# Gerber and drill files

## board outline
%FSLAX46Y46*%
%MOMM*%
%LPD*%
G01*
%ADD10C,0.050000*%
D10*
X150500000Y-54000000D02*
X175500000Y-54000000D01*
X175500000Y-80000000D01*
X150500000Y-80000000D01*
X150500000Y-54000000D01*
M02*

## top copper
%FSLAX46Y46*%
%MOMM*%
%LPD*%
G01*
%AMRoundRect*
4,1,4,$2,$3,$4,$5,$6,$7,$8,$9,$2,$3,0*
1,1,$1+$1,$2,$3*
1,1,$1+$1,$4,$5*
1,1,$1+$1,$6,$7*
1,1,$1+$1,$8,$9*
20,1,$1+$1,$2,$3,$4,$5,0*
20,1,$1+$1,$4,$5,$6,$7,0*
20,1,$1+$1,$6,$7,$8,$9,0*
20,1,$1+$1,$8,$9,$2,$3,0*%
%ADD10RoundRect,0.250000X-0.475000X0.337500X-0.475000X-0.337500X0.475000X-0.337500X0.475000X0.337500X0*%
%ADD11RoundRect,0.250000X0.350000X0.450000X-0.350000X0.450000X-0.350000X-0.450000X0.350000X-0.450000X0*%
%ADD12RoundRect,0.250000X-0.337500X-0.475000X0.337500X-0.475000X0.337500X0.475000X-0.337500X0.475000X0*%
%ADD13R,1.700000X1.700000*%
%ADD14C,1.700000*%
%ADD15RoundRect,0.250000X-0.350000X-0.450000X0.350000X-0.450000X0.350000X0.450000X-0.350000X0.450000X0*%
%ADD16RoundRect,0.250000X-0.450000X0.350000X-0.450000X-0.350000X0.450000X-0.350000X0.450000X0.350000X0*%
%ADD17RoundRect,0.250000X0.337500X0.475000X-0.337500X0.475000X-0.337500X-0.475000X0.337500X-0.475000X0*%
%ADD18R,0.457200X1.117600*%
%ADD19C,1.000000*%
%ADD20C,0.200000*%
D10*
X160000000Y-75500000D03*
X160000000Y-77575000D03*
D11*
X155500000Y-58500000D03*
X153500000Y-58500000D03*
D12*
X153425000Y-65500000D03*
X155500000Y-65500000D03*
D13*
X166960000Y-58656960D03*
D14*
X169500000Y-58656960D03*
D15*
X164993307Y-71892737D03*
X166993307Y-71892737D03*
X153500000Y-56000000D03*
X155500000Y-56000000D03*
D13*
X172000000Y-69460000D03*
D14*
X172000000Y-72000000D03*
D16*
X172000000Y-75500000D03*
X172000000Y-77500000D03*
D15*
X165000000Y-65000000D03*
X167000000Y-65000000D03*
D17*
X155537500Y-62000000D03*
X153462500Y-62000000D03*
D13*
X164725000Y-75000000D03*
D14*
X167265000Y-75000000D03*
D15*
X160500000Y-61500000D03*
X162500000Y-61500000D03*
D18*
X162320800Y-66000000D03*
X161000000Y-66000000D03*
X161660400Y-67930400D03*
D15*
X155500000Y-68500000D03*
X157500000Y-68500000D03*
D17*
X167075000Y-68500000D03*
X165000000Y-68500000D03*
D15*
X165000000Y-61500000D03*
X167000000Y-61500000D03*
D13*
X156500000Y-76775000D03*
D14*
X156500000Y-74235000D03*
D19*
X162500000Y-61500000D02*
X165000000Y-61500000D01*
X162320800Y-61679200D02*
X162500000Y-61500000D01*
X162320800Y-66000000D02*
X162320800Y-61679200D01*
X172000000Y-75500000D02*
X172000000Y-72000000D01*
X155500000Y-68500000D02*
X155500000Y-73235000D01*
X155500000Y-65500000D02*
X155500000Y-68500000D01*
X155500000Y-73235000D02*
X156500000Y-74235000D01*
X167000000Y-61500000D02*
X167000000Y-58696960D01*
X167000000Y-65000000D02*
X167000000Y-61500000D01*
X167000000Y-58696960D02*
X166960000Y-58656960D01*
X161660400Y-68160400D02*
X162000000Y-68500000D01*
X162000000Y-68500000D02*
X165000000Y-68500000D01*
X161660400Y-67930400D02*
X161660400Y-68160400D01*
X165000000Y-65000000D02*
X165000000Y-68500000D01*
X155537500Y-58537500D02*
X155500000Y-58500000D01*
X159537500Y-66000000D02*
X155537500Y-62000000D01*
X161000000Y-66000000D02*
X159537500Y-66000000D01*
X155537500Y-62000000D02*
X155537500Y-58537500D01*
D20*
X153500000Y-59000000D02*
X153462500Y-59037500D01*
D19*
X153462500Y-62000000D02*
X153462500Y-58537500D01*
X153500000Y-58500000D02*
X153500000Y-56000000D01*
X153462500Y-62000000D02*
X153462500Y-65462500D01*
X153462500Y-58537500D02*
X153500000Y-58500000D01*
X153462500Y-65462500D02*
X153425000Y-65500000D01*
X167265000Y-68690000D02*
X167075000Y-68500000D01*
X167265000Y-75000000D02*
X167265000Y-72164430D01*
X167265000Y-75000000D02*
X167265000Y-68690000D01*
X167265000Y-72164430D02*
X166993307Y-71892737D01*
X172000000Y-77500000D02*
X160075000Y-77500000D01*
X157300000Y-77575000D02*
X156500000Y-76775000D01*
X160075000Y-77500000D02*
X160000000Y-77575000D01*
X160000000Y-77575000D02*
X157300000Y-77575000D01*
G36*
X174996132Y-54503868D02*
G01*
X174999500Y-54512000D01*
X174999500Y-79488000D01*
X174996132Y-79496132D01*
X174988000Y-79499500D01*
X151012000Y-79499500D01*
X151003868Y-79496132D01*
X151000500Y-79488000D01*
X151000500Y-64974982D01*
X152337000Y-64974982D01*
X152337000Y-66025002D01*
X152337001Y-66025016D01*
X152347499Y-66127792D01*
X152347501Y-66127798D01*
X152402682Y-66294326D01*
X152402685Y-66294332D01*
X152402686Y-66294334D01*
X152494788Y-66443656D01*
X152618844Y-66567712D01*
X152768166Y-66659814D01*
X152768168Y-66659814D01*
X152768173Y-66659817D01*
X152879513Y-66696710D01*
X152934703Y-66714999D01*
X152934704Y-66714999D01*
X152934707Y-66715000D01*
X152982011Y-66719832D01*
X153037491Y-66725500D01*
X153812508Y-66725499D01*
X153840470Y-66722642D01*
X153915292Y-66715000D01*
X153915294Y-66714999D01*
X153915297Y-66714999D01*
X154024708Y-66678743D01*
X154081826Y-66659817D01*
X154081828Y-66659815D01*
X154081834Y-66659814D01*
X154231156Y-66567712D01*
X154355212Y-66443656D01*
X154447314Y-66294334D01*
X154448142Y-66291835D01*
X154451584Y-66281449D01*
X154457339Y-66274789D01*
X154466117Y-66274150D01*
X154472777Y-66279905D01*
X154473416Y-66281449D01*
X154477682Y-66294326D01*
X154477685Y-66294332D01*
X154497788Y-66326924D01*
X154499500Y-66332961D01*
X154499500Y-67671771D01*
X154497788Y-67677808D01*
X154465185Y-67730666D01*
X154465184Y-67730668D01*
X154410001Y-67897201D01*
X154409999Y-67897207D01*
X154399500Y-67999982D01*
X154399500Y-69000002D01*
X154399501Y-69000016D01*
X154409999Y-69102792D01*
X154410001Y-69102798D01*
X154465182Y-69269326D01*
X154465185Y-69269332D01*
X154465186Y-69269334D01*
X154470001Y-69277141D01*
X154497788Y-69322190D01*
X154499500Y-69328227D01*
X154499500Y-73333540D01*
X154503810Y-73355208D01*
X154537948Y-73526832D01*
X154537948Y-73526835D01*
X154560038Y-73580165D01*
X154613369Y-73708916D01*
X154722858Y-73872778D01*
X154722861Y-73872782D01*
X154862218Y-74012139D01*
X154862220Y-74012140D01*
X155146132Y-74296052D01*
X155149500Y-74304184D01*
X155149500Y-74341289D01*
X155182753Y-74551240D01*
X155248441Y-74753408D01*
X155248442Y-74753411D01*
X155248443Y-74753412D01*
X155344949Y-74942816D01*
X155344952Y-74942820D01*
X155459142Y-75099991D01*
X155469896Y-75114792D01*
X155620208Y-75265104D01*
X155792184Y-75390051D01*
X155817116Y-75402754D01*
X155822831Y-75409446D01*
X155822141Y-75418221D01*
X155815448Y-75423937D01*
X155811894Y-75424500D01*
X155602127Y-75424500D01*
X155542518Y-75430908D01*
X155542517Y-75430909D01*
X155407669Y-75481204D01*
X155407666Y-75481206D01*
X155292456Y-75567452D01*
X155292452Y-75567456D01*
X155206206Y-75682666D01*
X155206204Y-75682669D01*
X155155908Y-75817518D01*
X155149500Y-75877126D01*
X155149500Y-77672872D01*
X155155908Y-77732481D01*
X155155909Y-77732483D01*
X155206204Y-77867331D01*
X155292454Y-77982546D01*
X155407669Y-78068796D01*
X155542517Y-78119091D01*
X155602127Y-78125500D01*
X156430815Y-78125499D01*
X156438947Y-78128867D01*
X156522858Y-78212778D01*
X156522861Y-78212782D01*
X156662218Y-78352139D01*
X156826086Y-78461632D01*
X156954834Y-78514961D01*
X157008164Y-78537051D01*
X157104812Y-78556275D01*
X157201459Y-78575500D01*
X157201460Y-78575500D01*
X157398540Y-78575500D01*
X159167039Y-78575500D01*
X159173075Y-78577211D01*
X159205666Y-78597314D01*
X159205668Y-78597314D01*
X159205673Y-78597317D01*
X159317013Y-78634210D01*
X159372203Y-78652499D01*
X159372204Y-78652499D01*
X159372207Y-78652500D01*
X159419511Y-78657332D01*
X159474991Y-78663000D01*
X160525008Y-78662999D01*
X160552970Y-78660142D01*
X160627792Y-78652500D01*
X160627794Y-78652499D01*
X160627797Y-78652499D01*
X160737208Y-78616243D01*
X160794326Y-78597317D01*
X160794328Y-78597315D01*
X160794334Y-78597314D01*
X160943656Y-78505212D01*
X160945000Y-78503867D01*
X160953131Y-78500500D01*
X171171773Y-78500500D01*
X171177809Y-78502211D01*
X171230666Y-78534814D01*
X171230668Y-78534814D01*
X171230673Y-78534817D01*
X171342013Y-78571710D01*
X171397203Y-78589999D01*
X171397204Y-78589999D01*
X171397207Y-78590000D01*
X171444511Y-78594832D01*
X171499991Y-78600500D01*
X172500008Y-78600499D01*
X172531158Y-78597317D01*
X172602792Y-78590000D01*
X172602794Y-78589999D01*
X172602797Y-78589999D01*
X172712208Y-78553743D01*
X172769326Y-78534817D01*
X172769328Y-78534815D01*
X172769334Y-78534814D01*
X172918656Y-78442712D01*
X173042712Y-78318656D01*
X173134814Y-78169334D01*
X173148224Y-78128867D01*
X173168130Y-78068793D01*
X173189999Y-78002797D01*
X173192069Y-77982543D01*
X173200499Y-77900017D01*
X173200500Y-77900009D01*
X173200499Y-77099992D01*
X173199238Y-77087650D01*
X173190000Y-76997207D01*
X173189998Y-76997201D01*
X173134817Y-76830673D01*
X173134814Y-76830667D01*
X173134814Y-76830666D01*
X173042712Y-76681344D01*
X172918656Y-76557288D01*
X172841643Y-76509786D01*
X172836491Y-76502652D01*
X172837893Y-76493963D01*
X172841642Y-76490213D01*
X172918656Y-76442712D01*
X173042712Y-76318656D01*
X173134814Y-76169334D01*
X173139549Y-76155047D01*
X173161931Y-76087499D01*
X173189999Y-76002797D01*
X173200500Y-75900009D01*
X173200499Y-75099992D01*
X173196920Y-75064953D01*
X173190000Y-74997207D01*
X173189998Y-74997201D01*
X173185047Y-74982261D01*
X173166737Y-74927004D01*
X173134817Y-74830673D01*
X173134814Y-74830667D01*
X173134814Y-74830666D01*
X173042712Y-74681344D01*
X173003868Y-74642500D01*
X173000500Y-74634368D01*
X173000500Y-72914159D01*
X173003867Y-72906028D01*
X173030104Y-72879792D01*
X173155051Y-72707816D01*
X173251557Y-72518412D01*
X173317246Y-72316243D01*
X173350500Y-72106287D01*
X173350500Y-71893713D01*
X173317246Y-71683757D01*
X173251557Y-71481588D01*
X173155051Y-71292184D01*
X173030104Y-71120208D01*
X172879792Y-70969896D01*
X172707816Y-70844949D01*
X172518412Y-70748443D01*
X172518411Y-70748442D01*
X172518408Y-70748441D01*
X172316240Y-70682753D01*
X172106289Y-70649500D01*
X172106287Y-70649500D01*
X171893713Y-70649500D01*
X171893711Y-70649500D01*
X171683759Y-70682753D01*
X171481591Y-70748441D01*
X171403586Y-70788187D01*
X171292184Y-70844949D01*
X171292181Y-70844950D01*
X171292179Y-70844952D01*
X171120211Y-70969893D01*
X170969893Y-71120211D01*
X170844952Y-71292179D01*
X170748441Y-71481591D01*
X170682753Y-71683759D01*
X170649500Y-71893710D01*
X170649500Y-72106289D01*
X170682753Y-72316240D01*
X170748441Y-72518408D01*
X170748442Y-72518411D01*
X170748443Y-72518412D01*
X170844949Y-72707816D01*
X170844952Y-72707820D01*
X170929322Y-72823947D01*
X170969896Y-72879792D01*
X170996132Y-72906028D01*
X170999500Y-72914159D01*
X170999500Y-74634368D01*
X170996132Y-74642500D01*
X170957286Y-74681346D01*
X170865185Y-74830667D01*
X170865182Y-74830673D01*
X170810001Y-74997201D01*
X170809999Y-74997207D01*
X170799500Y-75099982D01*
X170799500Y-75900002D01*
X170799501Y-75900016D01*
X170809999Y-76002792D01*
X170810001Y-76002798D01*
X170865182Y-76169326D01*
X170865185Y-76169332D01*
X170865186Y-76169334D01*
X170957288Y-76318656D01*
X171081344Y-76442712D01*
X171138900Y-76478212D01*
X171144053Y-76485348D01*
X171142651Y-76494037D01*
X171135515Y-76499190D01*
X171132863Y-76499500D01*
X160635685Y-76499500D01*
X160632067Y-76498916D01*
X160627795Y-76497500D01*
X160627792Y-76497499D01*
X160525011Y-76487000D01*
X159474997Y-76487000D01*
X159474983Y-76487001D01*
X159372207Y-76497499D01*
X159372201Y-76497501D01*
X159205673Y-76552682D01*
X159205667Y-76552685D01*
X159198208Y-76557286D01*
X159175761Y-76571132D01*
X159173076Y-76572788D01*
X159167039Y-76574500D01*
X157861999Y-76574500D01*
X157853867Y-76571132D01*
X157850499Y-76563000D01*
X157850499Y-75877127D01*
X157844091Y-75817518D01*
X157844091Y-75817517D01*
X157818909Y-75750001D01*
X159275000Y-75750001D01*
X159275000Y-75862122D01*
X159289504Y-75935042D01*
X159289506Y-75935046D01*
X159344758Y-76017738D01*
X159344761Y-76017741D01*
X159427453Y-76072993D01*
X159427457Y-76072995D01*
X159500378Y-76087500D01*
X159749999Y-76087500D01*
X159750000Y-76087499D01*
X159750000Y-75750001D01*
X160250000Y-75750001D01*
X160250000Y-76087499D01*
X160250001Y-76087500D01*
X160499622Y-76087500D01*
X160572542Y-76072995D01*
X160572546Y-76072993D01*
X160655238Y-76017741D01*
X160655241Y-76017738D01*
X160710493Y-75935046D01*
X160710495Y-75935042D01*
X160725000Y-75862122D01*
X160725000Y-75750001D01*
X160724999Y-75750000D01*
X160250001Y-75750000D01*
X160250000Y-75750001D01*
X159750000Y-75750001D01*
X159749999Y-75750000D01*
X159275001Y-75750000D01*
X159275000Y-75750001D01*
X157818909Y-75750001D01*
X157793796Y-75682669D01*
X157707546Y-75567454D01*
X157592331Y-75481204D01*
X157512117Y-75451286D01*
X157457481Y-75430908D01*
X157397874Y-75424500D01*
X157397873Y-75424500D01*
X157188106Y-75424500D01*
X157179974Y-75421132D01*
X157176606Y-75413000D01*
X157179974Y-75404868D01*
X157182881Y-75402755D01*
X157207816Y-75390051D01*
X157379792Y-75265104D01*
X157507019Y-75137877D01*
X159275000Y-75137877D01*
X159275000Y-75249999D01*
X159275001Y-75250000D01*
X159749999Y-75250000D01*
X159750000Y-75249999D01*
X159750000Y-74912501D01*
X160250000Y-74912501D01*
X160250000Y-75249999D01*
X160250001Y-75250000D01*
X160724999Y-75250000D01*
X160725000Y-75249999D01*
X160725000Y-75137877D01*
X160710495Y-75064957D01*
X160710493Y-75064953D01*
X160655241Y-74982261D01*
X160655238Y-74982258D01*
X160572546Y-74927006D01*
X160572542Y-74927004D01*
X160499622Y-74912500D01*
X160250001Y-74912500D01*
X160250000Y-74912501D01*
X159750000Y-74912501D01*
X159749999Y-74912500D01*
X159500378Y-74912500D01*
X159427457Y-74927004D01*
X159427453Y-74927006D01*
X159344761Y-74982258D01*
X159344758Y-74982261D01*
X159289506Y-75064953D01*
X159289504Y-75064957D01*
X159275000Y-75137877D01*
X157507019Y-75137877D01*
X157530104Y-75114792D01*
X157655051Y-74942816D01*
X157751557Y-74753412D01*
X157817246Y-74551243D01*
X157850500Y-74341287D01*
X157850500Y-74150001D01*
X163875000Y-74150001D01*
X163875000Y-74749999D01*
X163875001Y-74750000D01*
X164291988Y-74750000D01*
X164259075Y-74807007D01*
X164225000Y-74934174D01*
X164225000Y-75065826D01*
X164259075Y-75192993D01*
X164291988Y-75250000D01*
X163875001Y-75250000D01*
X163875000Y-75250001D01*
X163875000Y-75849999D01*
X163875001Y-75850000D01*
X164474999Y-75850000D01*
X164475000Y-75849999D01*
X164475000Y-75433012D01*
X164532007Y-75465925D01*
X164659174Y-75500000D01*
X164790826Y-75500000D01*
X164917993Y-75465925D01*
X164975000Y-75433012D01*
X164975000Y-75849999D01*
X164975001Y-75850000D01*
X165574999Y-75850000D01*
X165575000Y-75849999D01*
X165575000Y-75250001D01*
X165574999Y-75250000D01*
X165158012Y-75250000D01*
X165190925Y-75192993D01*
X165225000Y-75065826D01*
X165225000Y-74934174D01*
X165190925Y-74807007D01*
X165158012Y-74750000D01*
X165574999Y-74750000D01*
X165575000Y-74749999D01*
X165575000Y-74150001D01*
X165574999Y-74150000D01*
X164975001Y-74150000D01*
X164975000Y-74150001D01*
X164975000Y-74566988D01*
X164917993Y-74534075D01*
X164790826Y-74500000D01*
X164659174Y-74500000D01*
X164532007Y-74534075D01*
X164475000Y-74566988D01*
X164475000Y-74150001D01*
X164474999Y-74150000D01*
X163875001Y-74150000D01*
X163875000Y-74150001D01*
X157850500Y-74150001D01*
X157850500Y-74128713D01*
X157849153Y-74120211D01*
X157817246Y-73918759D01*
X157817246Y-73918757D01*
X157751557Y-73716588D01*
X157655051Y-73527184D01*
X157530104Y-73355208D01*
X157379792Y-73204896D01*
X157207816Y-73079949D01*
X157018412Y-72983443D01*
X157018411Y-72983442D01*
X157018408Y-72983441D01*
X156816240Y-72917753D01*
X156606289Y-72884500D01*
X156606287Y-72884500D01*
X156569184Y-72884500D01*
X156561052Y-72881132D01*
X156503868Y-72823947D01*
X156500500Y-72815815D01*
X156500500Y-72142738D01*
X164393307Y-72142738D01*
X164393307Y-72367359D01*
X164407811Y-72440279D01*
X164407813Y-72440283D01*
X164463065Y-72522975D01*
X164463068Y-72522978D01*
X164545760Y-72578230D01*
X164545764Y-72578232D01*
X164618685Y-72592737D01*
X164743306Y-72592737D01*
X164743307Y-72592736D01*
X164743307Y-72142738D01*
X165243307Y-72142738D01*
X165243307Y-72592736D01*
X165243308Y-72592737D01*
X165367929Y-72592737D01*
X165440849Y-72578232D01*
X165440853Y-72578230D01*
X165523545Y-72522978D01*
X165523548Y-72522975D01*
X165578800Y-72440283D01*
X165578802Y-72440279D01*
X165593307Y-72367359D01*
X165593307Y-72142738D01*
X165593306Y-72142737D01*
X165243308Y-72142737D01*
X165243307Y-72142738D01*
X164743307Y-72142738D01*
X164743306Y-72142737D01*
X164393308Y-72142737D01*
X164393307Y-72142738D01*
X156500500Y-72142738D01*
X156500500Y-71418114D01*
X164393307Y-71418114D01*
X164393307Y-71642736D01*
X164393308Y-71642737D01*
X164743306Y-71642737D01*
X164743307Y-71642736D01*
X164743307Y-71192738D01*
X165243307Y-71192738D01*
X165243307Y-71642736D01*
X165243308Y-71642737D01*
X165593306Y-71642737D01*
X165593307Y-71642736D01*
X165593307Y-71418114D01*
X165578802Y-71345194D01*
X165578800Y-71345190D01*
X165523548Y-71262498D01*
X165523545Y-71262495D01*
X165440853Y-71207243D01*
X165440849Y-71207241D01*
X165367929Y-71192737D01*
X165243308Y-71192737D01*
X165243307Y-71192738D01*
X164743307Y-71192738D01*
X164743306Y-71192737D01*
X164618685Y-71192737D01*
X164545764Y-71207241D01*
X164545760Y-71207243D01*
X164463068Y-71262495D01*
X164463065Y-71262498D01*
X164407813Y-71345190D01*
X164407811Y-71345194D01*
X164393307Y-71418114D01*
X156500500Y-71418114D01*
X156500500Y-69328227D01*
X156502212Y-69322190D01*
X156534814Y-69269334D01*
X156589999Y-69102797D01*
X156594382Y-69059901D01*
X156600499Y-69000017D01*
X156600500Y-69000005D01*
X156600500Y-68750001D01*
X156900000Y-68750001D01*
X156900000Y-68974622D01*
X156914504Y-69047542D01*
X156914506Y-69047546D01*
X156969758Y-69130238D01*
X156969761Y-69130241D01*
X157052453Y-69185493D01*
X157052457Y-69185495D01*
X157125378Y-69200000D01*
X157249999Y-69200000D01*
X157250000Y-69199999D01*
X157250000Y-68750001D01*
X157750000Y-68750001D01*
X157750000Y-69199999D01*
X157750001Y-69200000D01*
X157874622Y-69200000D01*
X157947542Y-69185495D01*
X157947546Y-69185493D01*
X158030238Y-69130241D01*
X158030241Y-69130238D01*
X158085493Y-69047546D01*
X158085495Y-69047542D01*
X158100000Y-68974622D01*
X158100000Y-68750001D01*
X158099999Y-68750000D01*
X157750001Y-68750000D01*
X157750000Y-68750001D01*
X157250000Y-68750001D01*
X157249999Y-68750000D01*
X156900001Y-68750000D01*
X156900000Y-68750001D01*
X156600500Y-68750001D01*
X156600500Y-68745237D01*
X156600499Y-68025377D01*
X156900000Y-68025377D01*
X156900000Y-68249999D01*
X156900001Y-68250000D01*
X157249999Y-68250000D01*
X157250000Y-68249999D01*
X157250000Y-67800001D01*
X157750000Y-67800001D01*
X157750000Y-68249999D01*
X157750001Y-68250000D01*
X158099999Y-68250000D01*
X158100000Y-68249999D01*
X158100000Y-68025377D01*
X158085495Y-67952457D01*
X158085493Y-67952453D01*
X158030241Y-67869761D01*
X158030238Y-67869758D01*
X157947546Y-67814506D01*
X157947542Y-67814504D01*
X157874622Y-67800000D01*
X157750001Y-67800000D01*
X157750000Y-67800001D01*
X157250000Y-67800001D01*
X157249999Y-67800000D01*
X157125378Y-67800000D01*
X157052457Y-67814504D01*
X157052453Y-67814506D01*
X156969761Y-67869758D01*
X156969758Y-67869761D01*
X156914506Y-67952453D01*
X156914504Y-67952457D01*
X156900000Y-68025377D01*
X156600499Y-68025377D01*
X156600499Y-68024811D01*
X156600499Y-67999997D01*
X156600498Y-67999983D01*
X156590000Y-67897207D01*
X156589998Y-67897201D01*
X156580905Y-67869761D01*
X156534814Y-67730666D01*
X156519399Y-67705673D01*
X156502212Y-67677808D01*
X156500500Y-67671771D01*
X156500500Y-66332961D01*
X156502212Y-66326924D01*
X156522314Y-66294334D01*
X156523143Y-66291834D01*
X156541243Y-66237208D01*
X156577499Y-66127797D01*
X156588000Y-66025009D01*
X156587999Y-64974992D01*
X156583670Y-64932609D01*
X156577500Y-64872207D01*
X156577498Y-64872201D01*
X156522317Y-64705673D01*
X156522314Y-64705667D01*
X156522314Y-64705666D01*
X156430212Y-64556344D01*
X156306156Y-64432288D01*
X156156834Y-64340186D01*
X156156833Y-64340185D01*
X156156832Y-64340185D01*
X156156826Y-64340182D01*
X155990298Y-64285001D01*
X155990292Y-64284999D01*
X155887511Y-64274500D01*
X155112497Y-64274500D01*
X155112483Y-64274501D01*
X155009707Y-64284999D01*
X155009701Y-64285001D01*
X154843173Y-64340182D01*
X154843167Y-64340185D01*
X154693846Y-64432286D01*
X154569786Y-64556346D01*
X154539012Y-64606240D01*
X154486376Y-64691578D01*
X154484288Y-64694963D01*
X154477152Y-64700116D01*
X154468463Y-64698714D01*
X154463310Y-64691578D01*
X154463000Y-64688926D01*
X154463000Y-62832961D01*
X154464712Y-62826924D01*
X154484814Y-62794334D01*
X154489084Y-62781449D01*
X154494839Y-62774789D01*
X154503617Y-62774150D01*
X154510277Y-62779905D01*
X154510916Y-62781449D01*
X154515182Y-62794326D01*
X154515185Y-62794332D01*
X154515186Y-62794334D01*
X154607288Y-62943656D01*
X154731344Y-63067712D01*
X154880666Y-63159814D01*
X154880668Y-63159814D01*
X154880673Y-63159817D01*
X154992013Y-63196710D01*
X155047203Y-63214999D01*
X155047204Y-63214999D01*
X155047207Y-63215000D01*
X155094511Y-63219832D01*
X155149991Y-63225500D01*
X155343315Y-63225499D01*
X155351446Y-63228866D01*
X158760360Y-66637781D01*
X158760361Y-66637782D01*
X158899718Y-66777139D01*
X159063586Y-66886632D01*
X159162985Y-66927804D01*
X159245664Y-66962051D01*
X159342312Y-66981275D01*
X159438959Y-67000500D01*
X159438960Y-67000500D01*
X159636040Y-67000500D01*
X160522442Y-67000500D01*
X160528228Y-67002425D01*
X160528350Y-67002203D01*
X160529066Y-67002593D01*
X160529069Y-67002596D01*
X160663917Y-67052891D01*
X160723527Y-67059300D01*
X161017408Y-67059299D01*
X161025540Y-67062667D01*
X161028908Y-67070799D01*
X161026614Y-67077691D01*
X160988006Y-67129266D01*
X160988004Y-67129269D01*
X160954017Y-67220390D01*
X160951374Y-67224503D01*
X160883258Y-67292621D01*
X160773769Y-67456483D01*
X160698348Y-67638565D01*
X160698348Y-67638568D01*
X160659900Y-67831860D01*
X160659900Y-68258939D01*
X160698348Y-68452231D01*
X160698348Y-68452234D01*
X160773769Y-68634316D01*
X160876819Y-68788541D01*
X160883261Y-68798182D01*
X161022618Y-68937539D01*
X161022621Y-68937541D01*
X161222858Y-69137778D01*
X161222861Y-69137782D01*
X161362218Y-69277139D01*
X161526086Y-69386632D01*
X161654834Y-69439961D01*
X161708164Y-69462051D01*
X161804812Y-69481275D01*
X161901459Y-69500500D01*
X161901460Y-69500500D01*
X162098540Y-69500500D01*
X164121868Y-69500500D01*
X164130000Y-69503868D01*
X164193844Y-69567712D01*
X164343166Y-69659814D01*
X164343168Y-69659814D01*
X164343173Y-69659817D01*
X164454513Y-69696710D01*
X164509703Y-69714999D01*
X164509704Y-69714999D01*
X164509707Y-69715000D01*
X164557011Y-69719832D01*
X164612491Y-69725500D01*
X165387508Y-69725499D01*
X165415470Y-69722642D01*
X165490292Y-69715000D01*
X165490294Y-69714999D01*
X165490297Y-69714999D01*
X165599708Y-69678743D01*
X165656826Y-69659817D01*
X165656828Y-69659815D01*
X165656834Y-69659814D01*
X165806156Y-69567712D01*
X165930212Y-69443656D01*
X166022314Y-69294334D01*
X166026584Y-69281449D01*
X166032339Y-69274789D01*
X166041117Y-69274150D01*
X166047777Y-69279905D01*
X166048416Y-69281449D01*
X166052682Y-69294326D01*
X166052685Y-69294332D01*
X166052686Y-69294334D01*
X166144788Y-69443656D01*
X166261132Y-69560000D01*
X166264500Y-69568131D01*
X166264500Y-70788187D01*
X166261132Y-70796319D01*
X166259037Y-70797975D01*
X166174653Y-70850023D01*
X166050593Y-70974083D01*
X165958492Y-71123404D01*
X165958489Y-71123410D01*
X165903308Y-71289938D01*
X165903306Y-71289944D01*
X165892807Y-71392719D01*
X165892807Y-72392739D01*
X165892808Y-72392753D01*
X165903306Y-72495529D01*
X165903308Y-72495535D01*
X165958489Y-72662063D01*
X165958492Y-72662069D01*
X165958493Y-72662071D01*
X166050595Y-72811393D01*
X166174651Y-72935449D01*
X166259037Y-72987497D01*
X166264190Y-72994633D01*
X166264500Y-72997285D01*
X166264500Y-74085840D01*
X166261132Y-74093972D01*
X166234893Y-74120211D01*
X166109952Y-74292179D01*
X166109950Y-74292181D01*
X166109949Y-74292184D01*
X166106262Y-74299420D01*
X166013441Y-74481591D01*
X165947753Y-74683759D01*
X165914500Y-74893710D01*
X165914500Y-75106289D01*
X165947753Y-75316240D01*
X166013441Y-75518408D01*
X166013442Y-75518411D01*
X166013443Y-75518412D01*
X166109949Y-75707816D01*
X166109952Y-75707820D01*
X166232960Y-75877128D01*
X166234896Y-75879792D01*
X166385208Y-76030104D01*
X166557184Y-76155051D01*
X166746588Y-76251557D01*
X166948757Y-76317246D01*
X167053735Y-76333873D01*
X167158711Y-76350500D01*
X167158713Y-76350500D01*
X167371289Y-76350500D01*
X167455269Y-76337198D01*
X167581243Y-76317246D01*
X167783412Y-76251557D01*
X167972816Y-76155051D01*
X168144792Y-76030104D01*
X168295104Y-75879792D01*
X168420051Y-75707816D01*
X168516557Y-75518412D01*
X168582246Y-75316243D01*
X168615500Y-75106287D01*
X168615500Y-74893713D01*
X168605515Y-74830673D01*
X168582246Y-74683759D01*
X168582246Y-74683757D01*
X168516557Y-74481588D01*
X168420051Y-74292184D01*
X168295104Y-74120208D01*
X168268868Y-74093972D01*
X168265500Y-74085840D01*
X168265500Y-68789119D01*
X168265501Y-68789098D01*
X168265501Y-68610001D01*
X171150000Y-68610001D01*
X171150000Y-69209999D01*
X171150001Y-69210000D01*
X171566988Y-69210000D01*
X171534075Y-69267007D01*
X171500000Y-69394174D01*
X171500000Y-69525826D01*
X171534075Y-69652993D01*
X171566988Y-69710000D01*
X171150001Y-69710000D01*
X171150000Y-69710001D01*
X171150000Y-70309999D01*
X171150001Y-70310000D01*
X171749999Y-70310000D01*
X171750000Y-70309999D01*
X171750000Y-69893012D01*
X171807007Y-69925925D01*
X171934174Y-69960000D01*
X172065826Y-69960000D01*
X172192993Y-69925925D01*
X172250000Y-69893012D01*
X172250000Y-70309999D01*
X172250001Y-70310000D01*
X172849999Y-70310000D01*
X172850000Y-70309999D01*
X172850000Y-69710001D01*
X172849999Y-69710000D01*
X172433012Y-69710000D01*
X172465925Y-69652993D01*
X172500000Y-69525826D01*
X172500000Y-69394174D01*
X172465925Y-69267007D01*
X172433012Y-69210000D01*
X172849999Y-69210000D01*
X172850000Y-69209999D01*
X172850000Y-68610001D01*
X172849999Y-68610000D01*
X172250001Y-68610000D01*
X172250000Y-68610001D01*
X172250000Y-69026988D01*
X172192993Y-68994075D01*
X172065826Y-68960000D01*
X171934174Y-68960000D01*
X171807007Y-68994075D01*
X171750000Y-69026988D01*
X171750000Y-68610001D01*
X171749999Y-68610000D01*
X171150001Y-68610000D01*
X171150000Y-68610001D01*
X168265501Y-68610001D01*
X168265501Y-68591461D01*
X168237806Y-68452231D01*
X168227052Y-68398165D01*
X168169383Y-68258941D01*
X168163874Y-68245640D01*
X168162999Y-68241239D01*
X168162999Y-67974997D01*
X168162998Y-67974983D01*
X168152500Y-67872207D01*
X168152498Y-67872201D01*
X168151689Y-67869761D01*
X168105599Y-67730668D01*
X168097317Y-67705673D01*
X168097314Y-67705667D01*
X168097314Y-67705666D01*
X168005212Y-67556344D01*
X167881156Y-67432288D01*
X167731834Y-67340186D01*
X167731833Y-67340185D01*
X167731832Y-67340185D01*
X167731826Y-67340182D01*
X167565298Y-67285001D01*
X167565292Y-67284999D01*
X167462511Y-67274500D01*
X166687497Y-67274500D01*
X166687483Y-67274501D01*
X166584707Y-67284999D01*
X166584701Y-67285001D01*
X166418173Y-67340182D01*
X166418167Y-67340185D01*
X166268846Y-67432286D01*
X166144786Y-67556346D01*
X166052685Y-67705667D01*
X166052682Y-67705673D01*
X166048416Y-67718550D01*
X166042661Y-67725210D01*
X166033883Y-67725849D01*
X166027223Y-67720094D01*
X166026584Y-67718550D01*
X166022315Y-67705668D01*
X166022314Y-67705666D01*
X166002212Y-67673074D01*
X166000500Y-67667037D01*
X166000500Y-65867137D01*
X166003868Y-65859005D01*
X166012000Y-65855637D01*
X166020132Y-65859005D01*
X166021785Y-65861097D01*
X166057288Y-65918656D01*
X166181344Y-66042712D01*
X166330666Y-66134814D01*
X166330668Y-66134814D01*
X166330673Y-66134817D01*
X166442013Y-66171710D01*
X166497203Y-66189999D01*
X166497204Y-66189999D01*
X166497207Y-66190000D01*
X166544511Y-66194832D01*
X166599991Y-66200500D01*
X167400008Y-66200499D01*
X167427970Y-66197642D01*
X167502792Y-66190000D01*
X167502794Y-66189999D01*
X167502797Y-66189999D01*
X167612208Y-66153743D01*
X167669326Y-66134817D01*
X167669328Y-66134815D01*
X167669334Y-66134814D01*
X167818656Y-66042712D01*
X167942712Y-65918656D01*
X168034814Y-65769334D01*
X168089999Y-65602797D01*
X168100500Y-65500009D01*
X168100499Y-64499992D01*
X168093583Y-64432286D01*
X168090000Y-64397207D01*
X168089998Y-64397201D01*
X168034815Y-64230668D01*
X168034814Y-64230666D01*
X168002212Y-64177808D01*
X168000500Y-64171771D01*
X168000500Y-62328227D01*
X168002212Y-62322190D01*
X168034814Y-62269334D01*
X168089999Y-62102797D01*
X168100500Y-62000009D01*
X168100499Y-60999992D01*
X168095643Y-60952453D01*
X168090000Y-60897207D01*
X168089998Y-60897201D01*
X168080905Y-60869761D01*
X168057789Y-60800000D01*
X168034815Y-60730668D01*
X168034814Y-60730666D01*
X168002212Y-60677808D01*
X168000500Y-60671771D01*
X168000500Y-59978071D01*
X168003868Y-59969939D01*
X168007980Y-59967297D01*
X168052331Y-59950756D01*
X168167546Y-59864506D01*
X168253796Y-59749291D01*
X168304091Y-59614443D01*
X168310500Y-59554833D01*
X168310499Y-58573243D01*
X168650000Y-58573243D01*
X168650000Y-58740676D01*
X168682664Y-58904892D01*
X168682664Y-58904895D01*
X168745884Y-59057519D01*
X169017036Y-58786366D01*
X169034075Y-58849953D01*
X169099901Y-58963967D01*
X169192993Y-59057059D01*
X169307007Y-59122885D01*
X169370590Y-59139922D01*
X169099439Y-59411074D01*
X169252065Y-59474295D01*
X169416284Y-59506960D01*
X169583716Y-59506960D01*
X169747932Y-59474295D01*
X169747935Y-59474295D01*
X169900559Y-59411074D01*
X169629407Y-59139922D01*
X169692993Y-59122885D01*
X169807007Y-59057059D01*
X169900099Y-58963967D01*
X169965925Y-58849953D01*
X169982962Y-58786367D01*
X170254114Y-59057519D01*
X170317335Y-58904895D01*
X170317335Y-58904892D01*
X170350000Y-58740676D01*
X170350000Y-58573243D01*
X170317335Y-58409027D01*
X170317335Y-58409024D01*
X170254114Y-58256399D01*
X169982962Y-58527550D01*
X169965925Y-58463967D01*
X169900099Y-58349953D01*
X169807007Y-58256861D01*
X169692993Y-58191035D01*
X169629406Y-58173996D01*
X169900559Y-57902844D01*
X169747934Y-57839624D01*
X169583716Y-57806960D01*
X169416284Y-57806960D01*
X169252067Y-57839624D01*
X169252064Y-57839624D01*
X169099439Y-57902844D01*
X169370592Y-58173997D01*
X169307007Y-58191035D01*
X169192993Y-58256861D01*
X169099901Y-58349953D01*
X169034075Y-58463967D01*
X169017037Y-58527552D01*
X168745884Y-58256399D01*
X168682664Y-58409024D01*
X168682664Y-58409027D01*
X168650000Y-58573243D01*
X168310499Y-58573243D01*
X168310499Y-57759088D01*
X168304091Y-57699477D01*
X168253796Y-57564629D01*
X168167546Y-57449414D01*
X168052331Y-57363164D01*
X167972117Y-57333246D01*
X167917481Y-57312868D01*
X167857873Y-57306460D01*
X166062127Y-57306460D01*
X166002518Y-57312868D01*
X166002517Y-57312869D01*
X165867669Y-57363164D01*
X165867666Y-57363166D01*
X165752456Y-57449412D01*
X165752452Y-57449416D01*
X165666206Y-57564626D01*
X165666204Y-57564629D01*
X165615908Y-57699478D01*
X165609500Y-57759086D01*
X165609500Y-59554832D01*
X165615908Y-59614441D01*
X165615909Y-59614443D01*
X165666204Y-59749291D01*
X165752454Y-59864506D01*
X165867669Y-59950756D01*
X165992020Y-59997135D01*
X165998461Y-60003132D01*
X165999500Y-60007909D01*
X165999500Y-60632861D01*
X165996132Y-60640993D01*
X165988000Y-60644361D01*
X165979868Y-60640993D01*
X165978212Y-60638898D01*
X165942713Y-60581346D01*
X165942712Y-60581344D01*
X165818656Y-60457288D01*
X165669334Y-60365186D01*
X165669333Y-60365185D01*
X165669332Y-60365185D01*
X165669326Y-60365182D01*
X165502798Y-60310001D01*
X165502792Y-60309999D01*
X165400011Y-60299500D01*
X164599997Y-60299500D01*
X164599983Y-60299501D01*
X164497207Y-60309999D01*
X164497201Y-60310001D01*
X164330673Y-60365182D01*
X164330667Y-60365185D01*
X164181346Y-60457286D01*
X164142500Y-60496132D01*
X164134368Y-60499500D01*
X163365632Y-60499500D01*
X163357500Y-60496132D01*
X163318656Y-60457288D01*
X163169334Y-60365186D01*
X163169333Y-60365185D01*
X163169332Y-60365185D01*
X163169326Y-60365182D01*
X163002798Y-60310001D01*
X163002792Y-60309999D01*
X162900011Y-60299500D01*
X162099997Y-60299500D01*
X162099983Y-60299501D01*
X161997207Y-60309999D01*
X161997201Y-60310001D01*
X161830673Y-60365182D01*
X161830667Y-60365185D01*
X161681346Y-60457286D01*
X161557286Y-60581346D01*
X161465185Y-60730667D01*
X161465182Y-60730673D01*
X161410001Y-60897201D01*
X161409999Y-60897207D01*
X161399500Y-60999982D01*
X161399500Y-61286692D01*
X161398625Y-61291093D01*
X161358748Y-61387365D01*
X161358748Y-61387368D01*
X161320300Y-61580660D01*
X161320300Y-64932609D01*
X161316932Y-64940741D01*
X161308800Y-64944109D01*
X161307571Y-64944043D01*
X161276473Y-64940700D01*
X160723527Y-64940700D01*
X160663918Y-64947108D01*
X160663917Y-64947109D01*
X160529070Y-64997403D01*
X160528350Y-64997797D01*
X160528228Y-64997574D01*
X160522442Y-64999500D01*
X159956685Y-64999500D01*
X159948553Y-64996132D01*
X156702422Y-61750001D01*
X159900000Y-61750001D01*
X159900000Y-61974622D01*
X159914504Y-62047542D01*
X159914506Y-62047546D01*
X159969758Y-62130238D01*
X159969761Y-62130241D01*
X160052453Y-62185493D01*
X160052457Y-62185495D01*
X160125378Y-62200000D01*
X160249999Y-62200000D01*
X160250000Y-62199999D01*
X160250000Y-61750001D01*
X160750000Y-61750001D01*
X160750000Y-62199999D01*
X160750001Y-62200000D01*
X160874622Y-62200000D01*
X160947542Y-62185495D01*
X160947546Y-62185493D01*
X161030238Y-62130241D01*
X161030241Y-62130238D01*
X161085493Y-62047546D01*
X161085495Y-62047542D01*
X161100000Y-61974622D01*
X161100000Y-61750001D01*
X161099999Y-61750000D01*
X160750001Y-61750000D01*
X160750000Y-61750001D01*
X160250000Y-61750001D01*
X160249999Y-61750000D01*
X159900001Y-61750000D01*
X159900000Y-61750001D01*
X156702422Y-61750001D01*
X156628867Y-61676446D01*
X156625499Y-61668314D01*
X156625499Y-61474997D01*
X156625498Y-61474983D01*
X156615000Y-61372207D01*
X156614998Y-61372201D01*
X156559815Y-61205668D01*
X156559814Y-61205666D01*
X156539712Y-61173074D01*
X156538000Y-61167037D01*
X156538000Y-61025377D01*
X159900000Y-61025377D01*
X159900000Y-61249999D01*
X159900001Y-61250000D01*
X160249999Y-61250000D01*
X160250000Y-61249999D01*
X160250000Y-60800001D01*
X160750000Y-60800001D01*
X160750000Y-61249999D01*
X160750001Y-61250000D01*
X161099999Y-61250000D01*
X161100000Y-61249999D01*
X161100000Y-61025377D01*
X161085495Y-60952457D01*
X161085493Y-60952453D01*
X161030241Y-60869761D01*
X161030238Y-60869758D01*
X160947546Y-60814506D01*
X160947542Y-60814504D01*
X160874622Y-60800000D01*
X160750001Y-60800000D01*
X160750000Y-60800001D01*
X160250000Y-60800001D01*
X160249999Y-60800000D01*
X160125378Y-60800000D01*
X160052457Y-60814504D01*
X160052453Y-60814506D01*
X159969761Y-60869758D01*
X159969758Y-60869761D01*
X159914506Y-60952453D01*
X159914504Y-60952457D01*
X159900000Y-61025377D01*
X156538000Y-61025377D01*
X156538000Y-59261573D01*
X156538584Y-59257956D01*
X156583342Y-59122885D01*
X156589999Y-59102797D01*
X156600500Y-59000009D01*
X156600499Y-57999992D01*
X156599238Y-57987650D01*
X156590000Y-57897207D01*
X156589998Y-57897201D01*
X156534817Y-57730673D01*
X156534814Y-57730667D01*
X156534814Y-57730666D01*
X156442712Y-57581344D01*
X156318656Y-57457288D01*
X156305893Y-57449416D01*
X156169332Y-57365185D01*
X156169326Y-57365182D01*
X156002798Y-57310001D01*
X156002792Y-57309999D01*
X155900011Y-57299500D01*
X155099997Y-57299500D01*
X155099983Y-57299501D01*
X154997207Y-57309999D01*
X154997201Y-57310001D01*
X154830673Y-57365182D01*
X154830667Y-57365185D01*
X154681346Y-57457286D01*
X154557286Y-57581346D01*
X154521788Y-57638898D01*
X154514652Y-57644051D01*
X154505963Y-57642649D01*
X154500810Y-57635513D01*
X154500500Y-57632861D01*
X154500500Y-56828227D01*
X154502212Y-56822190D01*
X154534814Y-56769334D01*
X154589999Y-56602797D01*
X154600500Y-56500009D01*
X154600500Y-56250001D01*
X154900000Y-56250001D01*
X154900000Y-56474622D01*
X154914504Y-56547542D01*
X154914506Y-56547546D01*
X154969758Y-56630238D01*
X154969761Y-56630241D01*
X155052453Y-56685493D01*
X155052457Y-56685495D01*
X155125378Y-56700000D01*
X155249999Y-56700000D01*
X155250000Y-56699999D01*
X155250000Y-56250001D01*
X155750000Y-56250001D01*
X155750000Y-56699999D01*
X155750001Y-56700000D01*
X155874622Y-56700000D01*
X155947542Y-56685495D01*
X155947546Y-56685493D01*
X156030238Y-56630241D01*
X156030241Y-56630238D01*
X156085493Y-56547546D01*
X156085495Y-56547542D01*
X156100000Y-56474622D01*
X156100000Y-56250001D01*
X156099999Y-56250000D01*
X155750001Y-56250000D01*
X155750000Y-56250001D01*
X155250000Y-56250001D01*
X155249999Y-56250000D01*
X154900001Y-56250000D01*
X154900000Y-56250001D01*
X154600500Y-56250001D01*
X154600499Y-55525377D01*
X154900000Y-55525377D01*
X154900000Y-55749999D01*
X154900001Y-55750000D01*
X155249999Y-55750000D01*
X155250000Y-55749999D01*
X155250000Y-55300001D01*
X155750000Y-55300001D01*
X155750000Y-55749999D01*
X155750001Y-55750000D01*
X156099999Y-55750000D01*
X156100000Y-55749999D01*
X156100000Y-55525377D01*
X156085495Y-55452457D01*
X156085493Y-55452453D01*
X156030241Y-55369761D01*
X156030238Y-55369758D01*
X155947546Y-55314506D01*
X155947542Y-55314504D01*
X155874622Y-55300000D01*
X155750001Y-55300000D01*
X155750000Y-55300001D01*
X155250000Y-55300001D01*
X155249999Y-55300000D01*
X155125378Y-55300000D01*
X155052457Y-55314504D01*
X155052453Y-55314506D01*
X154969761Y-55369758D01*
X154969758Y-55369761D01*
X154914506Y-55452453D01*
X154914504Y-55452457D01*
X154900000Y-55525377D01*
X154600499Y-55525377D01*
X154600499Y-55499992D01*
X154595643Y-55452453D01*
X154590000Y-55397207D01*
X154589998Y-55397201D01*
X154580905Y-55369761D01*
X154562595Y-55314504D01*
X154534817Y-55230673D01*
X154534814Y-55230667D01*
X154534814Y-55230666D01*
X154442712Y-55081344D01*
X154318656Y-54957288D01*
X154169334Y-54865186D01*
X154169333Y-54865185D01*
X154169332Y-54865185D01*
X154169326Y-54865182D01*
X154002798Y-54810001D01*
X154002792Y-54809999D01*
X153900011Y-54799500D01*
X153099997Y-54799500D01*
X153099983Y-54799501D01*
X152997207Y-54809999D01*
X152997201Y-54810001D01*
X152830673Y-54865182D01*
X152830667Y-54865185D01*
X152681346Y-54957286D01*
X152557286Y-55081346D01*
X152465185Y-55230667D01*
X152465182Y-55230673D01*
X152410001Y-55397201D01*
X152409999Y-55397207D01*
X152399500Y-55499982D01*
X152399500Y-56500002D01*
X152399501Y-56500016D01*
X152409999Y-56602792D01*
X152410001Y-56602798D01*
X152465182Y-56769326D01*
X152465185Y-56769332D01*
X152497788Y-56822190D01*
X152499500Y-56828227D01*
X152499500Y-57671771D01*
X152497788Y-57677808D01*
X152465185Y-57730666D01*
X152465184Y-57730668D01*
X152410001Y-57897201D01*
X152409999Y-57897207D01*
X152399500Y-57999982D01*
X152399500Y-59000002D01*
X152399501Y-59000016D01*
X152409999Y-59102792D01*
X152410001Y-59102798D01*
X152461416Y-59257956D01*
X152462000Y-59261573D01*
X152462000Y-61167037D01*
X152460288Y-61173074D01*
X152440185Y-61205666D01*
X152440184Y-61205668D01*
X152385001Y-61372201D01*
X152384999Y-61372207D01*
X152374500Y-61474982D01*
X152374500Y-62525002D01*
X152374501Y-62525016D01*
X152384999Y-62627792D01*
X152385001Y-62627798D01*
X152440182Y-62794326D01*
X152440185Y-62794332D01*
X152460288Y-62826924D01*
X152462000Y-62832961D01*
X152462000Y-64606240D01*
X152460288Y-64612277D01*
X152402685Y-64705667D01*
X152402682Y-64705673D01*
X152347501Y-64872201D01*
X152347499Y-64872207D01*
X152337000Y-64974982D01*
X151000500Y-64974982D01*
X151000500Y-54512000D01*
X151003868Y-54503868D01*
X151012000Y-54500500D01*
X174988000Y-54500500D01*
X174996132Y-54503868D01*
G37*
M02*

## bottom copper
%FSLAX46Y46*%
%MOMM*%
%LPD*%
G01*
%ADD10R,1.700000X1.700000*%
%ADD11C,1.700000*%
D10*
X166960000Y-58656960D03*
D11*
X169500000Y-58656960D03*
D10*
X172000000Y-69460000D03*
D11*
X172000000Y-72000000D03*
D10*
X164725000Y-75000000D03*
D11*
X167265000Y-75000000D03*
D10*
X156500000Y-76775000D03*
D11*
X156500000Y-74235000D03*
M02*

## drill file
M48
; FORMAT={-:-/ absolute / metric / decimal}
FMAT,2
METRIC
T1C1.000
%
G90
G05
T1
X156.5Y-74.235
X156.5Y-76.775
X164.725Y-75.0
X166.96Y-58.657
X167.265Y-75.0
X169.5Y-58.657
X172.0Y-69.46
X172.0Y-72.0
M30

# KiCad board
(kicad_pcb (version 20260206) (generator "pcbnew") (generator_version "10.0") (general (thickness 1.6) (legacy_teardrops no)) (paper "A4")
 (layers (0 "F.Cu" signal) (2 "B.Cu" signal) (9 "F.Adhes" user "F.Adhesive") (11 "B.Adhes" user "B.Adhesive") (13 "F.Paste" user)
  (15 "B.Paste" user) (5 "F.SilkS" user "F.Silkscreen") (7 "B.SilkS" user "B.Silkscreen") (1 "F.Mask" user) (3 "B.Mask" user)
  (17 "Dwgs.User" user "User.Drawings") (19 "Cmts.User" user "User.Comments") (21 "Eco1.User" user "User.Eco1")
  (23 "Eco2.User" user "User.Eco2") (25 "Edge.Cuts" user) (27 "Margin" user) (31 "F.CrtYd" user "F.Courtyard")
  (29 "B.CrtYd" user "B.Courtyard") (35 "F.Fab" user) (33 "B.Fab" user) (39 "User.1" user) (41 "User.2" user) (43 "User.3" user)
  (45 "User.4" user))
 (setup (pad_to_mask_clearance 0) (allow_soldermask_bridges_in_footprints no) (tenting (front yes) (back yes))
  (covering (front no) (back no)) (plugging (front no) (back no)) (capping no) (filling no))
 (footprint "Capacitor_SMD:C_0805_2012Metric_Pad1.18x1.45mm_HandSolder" (layer "F.Cu") (at 160 76.5375 -90)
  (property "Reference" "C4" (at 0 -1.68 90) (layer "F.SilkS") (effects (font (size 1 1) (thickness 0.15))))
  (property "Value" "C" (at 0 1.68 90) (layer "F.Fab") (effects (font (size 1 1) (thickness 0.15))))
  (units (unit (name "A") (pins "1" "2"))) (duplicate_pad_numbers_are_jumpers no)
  (pad "1" smd roundrect (at -1.0375 0 270) (size 1.175 1.45) (layers "F.Cu" "F.Mask" "F.Paste") (roundrect_rratio 0.212766) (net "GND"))
  (pad "2" smd roundrect (at 1.0375 0 270) (size 1.175 1.45) (layers "F.Cu" "F.Mask" "F.Paste") (roundrect_rratio 0.212766)
   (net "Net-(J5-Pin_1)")))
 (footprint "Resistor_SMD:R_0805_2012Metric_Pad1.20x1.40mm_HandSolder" (layer "F.Cu") (at 154.5 58.5 180)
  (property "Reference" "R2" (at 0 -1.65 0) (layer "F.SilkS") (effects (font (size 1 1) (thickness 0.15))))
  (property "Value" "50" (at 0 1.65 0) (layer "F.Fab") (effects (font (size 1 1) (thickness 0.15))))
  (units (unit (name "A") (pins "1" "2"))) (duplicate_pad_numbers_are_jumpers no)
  (pad "1" smd roundrect (at -1 0 180) (size 1.2 1.4) (layers "F.Cu" "F.Mask" "F.Paste") (roundrect_rratio 0.208333) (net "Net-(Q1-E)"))
  (pad "2" smd roundrect (at 1 0 180) (size 1.2 1.4) (layers "F.Cu" "F.Mask" "F.Paste") (roundrect_rratio 0.208333) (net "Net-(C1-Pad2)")))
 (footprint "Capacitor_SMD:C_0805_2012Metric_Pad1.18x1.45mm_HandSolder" (layer "F.Cu") (at 154.4625 65.5)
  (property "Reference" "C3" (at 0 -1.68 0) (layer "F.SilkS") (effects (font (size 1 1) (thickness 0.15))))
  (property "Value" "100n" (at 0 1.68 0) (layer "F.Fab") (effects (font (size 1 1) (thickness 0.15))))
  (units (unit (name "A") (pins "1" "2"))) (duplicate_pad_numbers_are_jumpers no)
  (pad "1" smd roundrect (at -1.0375 0) (size 1.175 1.45) (layers "F.Cu" "F.Mask" "F.Paste") (roundrect_rratio 0.212766)
   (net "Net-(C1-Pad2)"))
  (pad "2" smd roundrect (at 1.0375 0) (size 1.175 1.45) (layers "F.Cu" "F.Mask" "F.Paste") (roundrect_rratio 0.212766)
   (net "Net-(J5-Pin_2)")))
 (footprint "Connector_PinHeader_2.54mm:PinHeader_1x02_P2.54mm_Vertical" (layer "F.Cu") (at 166.96 58.65696 90)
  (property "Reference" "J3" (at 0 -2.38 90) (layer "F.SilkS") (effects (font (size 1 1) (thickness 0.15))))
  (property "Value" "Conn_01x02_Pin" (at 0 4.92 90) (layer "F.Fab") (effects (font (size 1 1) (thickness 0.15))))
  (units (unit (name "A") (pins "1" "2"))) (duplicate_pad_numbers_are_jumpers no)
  (pad "1" thru_hole rect (at 0 0 90) (size 1.7 1.7) (drill 1) (layers "*.Cu" "*.Mask") (remove_unused_layers no) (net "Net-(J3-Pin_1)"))
  (pad "2" thru_hole circle (at 0 2.54 90) (size 1.7 1.7) (drill 1) (layers "*.Cu" "*.Mask") (remove_unused_layers no) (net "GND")))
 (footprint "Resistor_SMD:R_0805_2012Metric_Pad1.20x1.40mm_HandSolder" (layer "F.Cu") (at 165.993307 71.892737)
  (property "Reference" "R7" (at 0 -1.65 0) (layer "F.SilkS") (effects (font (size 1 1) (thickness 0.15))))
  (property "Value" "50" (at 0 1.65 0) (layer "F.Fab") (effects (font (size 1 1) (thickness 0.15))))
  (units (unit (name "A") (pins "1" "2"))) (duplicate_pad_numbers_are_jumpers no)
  (pad "1" smd roundrect (at -1 0) (size 1.2 1.4) (layers "F.Cu" "F.Mask" "F.Paste") (roundrect_rratio 0.208333) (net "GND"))
  (pad "2" smd roundrect (at 1 0) (size 1.2 1.4) (layers "F.Cu" "F.Mask" "F.Paste") (roundrect_rratio 0.208333) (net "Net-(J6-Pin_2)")))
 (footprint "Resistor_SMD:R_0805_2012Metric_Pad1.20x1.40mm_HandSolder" (layer "F.Cu") (at 154.5 56)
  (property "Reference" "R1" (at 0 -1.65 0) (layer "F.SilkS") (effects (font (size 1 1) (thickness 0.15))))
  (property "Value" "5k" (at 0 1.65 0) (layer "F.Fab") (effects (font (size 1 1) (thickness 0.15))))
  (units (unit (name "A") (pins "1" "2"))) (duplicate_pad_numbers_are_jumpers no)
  (pad "1" smd roundrect (at -1 0) (size 1.2 1.4) (layers "F.Cu" "F.Mask" "F.Paste") (roundrect_rratio 0.208333) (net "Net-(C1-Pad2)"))
  (pad "2" smd roundrect (at 1 0) (size 1.2 1.4) (layers "F.Cu" "F.Mask" "F.Paste") (roundrect_rratio 0.208333) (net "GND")))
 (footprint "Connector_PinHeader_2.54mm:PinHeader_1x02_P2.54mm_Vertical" (layer "F.Cu") (at 172 69.46)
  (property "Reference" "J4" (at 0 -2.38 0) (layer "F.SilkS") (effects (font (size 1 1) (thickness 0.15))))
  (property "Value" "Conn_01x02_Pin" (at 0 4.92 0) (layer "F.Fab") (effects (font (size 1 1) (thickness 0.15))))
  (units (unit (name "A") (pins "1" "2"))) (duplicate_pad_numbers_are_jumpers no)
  (pad "1" thru_hole rect (at 0 0) (size 1.7 1.7) (drill 1) (layers "*.Cu" "*.Mask") (remove_unused_layers no) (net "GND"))
  (pad "2" thru_hole circle (at 0 2.54) (size 1.7 1.7) (drill 1) (layers "*.Cu" "*.Mask") (remove_unused_layers no) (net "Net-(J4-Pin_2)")))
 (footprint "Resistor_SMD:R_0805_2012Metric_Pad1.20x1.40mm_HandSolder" (layer "F.Cu") (at 172 76.5 -90)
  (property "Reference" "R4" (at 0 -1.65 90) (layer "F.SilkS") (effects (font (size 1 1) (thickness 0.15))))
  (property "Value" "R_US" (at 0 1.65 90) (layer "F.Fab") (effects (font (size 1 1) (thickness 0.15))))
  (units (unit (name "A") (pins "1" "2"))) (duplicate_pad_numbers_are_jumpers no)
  (pad "1" smd roundrect (at -1 0 270) (size 1.2 1.4) (layers "F.Cu" "F.Mask" "F.Paste") (roundrect_rratio 0.208333) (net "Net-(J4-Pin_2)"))
  (pad "2" smd roundrect (at 1 0 270) (size 1.2 1.4) (layers "F.Cu" "F.Mask" "F.Paste") (roundrect_rratio 0.208333) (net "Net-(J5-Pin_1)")))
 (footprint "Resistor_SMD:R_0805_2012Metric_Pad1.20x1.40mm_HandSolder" (layer "F.Cu") (at 166 65)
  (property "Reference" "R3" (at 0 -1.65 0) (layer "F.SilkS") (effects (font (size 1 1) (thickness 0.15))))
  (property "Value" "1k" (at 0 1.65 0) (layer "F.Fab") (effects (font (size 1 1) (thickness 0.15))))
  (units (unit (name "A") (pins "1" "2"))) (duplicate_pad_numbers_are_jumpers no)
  (pad "1" smd roundrect (at -1 0) (size 1.2 1.4) (layers "F.Cu" "F.Mask" "F.Paste") (roundrect_rratio 0.208333) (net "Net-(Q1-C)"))
  (pad "2" smd roundrect (at 1 0) (size 1.2 1.4) (layers "F.Cu" "F.Mask" "F.Paste") (roundrect_rratio 0.208333) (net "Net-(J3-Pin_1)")))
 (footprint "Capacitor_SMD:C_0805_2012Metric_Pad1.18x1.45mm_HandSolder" (layer "F.Cu") (at 154.5 62 180)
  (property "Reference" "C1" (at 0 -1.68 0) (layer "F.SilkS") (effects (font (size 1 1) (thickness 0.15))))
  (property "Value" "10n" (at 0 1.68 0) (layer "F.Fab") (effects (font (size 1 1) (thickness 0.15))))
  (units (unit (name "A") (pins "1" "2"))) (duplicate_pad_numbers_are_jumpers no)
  (pad "1" smd roundrect (at -1.0375 0 180) (size 1.175 1.45) (layers "F.Cu" "F.Mask" "F.Paste") (roundrect_rratio 0.212766)
   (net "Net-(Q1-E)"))
  (pad "2" smd roundrect (at 1.0375 0 180) (size 1.175 1.45) (layers "F.Cu" "F.Mask" "F.Paste") (roundrect_rratio 0.212766)
   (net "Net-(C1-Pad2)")))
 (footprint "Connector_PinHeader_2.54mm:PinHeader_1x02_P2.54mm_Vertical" (layer "F.Cu") (at 164.725 75 90)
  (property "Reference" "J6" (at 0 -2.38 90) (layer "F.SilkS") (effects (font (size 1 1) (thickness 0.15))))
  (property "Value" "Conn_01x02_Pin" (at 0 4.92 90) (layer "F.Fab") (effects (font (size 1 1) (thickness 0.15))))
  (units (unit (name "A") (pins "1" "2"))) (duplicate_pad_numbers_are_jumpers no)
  (pad "1" thru_hole rect (at 0 0 90) (size 1.7 1.7) (drill 1) (layers "*.Cu" "*.Mask") (remove_unused_layers no) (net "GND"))
  (pad "2" thru_hole circle (at 0 2.54 90) (size 1.7 1.7) (drill 1) (layers "*.Cu" "*.Mask") (remove_unused_layers no)
   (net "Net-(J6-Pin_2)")))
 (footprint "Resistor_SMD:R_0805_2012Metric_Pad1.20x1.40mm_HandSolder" (layer "F.Cu") (at 161.5 61.5)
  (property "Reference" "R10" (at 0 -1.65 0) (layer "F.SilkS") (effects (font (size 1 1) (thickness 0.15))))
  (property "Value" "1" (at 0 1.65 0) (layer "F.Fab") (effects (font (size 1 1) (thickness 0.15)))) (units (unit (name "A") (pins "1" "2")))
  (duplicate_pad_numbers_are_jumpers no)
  (pad "1" smd roundrect (at -1 0) (size 1.2 1.4) (layers "F.Cu" "F.Mask" "F.Paste") (roundrect_rratio 0.208333) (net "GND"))
  (pad "2" smd roundrect (at 1 0) (size 1.2 1.4) (layers "F.Cu" "F.Mask" "F.Paste") (roundrect_rratio 0.208333) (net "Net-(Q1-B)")))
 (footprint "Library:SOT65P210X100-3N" (layer "F.Cu") (at 161.6604 66.9652 -90)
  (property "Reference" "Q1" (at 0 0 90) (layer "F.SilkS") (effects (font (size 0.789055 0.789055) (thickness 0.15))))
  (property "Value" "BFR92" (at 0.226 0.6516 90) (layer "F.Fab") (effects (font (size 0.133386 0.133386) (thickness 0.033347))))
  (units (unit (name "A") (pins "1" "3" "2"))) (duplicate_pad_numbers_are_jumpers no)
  (pad "1" smd rect (at -0.9652 -0.6604 270) (size 1.1176 0.4572) (layers "F.Cu" "F.Mask" "F.Paste") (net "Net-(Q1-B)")
   (solder_mask_margin 0.102))
  (pad "2" smd rect (at -0.9652 0.6604 270) (size 1.1176 0.4572) (layers "F.Cu" "F.Mask" "F.Paste") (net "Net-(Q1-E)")
   (solder_mask_margin 0.102))
  (pad "3" smd rect (at 0.9652 0 270) (size 1.1176 0.4572) (layers "F.Cu" "F.Mask" "F.Paste") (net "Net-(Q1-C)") (solder_mask_margin 0.102)))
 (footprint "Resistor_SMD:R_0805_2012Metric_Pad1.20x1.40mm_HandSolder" (layer "F.Cu") (at 156.5 68.5)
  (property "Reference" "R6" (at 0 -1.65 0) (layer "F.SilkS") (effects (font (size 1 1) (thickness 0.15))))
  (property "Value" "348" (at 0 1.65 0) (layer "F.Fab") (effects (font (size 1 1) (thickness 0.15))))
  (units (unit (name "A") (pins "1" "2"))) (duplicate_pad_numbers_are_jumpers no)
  (pad "1" smd roundrect (at -1 0) (size 1.2 1.4) (layers "F.Cu" "F.Mask" "F.Paste") (roundrect_rratio 0.208333) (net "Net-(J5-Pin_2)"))
  (pad "2" smd roundrect (at 1 0) (size 1.2 1.4) (layers "F.Cu" "F.Mask" "F.Paste") (roundrect_rratio 0.208333) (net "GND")))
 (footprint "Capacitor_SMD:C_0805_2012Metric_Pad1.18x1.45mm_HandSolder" (layer "F.Cu") (at 166.0375 68.5 180)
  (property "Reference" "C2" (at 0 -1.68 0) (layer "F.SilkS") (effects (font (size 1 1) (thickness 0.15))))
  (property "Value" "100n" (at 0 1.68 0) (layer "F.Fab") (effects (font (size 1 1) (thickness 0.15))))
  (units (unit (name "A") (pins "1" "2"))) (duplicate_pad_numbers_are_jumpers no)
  (pad "1" smd roundrect (at -1.0375 0 180) (size 1.175 1.45) (layers "F.Cu" "F.Mask" "F.Paste") (roundrect_rratio 0.212766)
   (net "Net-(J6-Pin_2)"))
  (pad "2" smd roundrect (at 1.0375 0 180) (size 1.175 1.45) (layers "F.Cu" "F.Mask" "F.Paste") (roundrect_rratio 0.212766)
   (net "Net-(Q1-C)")))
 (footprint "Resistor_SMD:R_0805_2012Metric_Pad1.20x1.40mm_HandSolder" (layer "F.Cu") (at 166 61.5)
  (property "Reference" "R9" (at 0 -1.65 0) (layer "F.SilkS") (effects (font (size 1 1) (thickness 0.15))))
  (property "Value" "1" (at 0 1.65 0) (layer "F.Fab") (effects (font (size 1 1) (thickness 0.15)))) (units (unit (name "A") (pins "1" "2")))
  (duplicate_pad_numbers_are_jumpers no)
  (pad "1" smd roundrect (at -1 0) (size 1.2 1.4) (layers "F.Cu" "F.Mask" "F.Paste") (roundrect_rratio 0.208333) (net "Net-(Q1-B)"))
  (pad "2" smd roundrect (at 1 0) (size 1.2 1.4) (layers "F.Cu" "F.Mask" "F.Paste") (roundrect_rratio 0.208333) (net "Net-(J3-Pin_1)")))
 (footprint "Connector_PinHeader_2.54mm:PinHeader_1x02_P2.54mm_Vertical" (layer "F.Cu") (at 156.5 76.775 180)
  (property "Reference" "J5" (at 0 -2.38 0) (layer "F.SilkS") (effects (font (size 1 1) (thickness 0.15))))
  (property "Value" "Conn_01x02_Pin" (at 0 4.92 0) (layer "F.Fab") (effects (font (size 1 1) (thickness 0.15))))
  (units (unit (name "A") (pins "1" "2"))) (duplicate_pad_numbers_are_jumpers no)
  (pad "1" thru_hole rect (at 0 0 180) (size 1.7 1.7) (drill 1) (layers "*.Cu" "*.Mask") (remove_unused_layers no) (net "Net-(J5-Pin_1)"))
  (pad "2" thru_hole circle (at 0 2.54 180) (size 1.7 1.7) (drill 1) (layers "*.Cu" "*.Mask") (remove_unused_layers no)
   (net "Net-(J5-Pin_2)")))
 (gr_rect (start 150.5 54) (end 175.5 80) (stroke (width 0.05) (type default)) (fill no) (layer "Edge.Cuts"))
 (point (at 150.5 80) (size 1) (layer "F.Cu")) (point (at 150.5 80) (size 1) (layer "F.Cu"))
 (segment (start 162.5 61.5) (end 165 61.5) (width 1) (layer "F.Cu") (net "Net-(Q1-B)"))
 (segment (start 162.3208 61.6792) (end 162.5 61.5) (width 1) (layer "F.Cu") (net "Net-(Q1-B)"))
 (segment (start 162.3208 66) (end 162.3208 61.6792) (width 1) (layer "F.Cu") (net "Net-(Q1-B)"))
 (segment (start 172 75.5) (end 172 72) (width 1) (layer "F.Cu") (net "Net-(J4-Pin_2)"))
 (segment (start 155.5 68.5) (end 155.5 73.235) (width 1) (layer "F.Cu") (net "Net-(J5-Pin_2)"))
 (segment (start 155.5 65.5) (end 155.5 68.5) (width 1) (layer "F.Cu") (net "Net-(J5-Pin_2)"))
 (segment (start 155.5 73.235) (end 156.5 74.235) (width 1) (layer "F.Cu") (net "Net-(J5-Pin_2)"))
 (segment (start 167 61.5) (end 167 58.69696) (width 1) (layer "F.Cu") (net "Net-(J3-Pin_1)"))
 (segment (start 167 65) (end 167 61.5) (width 1) (layer "F.Cu") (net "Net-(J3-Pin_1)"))
 (segment (start 167 58.69696) (end 166.96 58.65696) (width 1) (layer "F.Cu") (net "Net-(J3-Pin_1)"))
 (segment (start 161.6604 68.1604) (end 162 68.5) (width 1) (layer "F.Cu") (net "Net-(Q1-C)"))
 (segment (start 162 68.5) (end 165 68.5) (width 1) (layer "F.Cu") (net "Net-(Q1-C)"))
 (segment (start 161.6604 67.9304) (end 161.6604 68.1604) (width 1) (layer "F.Cu") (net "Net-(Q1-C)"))
 (segment (start 165 65) (end 165 68.5) (width 1) (layer "F.Cu") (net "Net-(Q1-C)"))
 (segment (start 155.5375 58.5375) (end 155.5 58.5) (width 1) (layer "F.Cu") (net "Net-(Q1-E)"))
 (segment (start 159.5375 66) (end 155.5375 62) (width 1) (layer "F.Cu") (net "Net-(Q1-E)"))
 (segment (start 161 66) (end 159.5375 66) (width 1) (layer "F.Cu") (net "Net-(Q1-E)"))
 (segment (start 155.5375 62) (end 155.5375 58.5375) (width 1) (layer "F.Cu") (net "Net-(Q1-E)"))
 (segment (start 153.5 59) (end 153.4625 59.0375) (width 0.2) (layer "F.Cu") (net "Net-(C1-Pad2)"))
 (segment (start 153.4625 62) (end 153.4625 58.5375) (width 1) (layer "F.Cu") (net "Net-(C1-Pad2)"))
 (segment (start 153.5 58.5) (end 153.5 56) (width 1) (layer "F.Cu") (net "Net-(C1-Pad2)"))
 (segment (start 153.4625 62) (end 153.4625 65.4625) (width 1) (layer "F.Cu") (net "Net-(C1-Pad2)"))
 (segment (start 153.4625 58.5375) (end 153.5 58.5) (width 1) (layer "F.Cu") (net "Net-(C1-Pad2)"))
 (segment (start 153.4625 65.4625) (end 153.425 65.5) (width 1) (layer "F.Cu") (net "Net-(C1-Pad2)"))
 (segment (start 167.265 68.69) (end 167.075 68.5) (width 1) (layer "F.Cu") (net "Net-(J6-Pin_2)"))
 (segment (start 167.265 75) (end 167.265 72.16443) (width 1) (layer "F.Cu") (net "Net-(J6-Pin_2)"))
 (segment (start 167.265 75) (end 167.265 68.69) (width 1) (layer "F.Cu") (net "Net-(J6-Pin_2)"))
 (segment (start 167.265 72.16443) (end 166.993307 71.892737) (width 1) (layer "F.Cu") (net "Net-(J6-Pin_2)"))
 (segment (start 172 77.5) (end 160.075 77.5) (width 1) (layer "F.Cu") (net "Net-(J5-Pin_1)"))
 (segment (start 157.3 77.575) (end 156.5 76.775) (width 1) (layer "F.Cu") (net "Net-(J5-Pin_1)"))
 (segment (start 160.075 77.5) (end 160 77.575) (width 1) (layer "F.Cu") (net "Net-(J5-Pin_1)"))
 (segment (start 160 77.575) (end 157.3 77.575) (width 1) (layer "F.Cu") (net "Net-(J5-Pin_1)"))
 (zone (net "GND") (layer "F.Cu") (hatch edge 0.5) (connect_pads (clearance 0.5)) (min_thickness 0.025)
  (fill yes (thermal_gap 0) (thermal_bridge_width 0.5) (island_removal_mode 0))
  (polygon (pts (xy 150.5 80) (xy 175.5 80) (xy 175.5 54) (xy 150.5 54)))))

